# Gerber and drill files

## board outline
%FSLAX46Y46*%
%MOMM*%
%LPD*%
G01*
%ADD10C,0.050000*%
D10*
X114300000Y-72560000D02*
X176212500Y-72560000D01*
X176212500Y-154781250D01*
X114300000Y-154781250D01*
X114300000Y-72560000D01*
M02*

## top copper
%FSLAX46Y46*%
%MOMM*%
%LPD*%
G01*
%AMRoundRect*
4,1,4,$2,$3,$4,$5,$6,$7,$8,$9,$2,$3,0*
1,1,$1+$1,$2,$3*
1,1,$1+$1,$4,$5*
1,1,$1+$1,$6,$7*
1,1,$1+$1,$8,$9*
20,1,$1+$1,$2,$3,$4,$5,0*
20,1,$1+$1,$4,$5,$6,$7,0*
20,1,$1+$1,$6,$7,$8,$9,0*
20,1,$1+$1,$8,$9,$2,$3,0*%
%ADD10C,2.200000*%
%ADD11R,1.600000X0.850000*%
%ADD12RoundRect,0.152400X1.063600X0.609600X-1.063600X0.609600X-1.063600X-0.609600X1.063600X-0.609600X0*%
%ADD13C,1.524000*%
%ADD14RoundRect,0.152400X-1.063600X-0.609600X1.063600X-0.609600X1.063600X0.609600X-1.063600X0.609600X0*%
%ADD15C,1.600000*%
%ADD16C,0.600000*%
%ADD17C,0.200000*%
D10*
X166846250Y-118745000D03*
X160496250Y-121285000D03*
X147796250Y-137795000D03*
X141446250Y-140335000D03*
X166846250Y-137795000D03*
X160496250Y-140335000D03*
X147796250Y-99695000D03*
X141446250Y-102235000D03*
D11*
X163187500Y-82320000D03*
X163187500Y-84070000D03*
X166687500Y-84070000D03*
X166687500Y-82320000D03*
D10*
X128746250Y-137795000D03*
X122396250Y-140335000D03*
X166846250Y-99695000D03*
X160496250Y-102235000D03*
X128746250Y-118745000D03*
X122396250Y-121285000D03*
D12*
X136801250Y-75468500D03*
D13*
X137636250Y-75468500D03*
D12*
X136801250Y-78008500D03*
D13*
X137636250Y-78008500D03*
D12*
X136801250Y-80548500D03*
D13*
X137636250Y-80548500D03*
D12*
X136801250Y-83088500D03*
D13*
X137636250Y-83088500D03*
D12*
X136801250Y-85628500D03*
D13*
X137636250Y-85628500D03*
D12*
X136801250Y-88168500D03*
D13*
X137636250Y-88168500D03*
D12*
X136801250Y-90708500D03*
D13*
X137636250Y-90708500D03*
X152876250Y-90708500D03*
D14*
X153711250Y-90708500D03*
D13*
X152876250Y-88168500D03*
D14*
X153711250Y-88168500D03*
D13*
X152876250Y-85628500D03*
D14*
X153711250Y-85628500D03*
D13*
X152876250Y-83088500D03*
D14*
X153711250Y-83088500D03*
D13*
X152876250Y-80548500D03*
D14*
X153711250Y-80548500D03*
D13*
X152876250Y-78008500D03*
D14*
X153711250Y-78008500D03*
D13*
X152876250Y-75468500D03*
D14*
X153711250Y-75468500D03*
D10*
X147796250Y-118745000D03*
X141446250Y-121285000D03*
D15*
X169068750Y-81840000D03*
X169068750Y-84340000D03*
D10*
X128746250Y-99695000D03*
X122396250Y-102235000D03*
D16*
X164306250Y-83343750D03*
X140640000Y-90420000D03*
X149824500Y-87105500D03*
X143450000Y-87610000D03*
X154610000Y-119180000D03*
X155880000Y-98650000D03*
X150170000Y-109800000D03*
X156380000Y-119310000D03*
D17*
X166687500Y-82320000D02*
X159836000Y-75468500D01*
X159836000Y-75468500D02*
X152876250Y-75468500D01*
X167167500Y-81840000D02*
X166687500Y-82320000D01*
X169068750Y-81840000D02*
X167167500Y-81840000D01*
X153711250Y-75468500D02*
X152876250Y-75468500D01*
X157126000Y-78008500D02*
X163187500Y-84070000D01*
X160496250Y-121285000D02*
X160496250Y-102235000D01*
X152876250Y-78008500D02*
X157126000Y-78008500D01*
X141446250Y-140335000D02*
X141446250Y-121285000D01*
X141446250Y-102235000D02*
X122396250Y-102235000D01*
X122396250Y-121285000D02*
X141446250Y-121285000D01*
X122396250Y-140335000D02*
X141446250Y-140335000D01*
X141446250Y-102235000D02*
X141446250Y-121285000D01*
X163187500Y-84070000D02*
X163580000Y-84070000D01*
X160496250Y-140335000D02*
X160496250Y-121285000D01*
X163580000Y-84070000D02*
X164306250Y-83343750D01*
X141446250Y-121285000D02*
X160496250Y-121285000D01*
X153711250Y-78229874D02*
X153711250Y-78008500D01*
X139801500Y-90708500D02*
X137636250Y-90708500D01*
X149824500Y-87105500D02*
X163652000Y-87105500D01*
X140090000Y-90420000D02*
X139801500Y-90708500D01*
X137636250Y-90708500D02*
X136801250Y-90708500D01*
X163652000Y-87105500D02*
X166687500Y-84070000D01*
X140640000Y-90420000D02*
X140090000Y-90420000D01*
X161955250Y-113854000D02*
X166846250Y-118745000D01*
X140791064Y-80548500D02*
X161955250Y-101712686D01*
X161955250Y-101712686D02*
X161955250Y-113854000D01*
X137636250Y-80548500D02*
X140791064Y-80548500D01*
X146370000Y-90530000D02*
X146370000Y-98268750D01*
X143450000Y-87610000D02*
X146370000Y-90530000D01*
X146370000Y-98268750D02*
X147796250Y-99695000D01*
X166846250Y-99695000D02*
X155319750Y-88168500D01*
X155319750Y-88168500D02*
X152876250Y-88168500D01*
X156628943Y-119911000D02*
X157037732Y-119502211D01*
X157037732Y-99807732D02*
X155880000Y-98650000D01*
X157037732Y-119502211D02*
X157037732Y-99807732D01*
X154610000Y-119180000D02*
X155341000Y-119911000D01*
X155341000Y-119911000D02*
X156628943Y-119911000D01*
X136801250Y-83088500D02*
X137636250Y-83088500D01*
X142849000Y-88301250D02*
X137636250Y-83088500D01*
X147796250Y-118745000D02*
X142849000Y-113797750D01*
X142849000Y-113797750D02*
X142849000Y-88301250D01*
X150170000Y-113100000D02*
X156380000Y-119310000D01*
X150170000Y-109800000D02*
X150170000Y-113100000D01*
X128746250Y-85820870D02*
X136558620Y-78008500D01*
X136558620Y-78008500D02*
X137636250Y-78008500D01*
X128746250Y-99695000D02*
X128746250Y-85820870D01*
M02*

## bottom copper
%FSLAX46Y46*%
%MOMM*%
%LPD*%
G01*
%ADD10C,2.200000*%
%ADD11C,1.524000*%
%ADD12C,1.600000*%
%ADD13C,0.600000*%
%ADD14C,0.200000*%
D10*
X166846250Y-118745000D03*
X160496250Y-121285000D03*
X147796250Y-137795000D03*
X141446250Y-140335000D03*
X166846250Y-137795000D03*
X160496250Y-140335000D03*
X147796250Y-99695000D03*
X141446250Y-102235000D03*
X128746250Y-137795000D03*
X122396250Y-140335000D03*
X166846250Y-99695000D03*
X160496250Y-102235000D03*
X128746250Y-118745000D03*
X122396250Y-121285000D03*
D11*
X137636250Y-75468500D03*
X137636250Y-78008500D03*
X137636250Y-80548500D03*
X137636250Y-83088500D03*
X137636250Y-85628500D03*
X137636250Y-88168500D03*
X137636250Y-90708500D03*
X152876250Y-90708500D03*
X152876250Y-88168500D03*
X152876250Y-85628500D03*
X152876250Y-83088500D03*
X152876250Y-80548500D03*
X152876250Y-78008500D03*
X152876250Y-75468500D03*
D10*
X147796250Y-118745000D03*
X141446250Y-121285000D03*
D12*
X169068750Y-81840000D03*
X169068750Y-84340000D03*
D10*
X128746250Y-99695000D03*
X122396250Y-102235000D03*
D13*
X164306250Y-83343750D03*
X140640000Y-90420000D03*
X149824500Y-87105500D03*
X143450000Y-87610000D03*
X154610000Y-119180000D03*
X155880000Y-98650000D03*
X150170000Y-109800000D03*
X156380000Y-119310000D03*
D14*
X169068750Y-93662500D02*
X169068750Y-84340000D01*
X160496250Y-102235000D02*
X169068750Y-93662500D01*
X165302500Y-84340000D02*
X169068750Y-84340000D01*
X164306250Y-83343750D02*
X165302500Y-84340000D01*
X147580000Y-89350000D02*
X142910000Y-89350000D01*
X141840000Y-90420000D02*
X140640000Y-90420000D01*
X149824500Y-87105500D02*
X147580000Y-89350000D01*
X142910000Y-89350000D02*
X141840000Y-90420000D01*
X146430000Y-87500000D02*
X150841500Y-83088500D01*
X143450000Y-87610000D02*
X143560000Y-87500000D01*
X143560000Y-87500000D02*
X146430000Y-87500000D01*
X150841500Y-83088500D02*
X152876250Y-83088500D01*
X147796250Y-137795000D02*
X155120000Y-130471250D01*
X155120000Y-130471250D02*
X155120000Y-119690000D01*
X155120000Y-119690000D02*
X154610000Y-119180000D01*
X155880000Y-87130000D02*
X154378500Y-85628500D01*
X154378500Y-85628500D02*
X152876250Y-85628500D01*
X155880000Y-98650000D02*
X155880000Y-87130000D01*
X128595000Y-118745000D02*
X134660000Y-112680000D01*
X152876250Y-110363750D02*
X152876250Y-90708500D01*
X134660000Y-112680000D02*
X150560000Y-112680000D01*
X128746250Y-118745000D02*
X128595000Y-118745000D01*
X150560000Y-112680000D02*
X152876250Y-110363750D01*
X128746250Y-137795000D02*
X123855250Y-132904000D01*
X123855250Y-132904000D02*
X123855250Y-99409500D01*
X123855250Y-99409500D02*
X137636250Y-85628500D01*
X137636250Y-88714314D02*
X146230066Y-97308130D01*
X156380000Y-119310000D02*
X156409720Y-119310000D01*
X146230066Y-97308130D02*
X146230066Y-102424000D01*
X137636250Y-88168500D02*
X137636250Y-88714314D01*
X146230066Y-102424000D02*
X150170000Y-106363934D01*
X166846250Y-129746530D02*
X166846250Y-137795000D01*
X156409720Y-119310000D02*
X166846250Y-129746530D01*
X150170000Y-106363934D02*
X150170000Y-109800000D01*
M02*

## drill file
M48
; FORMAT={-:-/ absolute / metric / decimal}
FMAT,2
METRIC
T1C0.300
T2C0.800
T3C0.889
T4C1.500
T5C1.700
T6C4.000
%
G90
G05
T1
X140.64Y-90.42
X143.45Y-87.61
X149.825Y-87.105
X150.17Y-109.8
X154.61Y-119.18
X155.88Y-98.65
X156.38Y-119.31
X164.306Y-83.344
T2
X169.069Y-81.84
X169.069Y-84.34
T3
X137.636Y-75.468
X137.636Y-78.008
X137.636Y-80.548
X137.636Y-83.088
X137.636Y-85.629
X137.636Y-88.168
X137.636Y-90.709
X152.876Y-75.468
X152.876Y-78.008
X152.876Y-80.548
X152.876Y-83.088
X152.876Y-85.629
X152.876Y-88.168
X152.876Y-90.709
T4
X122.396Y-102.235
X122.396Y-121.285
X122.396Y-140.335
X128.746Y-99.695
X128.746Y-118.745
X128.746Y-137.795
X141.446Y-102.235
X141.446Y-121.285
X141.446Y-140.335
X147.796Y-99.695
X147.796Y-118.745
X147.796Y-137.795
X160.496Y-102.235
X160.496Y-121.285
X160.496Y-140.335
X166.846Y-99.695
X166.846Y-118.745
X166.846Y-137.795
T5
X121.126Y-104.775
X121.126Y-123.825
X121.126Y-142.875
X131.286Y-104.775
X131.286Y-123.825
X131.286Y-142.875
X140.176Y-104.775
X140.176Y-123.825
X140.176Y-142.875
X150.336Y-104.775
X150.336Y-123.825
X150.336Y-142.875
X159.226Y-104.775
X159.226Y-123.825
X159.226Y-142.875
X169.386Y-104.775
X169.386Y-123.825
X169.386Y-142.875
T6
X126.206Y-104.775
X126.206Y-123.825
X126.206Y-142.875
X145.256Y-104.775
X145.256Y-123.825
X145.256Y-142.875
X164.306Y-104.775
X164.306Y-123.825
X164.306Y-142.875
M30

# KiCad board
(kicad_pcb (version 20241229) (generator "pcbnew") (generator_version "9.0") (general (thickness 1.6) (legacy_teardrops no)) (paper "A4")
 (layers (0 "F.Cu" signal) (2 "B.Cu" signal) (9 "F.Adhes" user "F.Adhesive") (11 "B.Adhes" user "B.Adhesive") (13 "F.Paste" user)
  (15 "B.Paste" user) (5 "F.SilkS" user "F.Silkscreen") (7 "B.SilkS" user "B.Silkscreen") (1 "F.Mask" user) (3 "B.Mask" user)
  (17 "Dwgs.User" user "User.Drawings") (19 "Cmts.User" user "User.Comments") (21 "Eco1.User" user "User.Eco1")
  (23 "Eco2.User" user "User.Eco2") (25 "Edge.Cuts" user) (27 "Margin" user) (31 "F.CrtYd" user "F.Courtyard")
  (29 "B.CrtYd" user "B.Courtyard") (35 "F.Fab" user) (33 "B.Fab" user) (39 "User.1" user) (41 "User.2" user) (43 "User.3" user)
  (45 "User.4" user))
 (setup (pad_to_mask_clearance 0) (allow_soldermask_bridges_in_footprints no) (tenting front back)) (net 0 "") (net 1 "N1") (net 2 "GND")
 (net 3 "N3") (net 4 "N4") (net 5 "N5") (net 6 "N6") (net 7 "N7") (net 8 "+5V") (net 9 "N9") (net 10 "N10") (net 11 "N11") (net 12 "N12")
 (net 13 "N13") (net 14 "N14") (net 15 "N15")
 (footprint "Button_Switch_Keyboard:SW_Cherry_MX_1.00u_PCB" (layer "F.Cu") (at 166.84625 118.745)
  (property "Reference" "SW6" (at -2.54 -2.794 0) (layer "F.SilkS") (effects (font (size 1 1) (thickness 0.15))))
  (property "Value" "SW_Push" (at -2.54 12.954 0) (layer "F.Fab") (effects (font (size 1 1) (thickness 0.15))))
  (pad "" np_thru_hole circle (at -7.62 5.08) (size 1.7 1.7) (drill 1.7) (layers "*.Cu" "*.Mask"))
  (pad "" np_thru_hole circle (at -2.54 5.08) (size 4 4) (drill 4) (layers "*.Cu" "*.Mask"))
  (pad "" np_thru_hole circle (at 2.54 5.08) (size 1.7 1.7) (drill 1.7) (layers "*.Cu" "*.Mask"))
  (pad "1" thru_hole circle (at 0 0) (size 2.2 2.2) (drill 1.5) (layers "*.Cu" "*.Mask") (remove_unused_layers no) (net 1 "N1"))
  (pad "2" thru_hole circle (at -6.35 2.54) (size 2.2 2.2) (drill 1.5) (layers "*.Cu" "*.Mask") (remove_unused_layers no) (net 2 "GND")))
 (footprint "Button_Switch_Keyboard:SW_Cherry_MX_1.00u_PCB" (layer "F.Cu") (at 147.79625 137.795)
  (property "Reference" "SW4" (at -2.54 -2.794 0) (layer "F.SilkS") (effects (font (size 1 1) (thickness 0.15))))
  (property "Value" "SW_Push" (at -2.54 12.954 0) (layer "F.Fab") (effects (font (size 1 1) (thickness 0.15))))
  (pad "" np_thru_hole circle (at -7.62 5.08) (size 1.7 1.7) (drill 1.7) (layers "*.Cu" "*.Mask"))
  (pad "" np_thru_hole circle (at -2.54 5.08) (size 4 4) (drill 4) (layers "*.Cu" "*.Mask"))
  (pad "" np_thru_hole circle (at 2.54 5.08) (size 1.7 1.7) (drill 1.7) (layers "*.Cu" "*.Mask"))
  (pad "1" thru_hole circle (at 0 0) (size 2.2 2.2) (drill 1.5) (layers "*.Cu" "*.Mask") (remove_unused_layers no) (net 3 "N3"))
  (pad "2" thru_hole circle (at -6.35 2.54) (size 2.2 2.2) (drill 1.5) (layers "*.Cu" "*.Mask") (remove_unused_layers no) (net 2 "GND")))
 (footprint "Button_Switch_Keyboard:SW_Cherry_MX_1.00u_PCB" (layer "F.Cu") (at 166.84625 137.795)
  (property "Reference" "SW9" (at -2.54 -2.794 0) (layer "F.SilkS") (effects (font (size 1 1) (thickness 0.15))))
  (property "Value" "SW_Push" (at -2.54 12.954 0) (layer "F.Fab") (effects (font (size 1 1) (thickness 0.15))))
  (pad "" np_thru_hole circle (at -7.62 5.08) (size 1.7 1.7) (drill 1.7) (layers "*.Cu" "*.Mask"))
  (pad "" np_thru_hole circle (at -2.54 5.08) (size 4 4) (drill 4) (layers "*.Cu" "*.Mask"))
  (pad "" np_thru_hole circle (at 2.54 5.08) (size 1.7 1.7) (drill 1.7) (layers "*.Cu" "*.Mask"))
  (pad "1" thru_hole circle (at 0 0) (size 2.2 2.2) (drill 1.5) (layers "*.Cu" "*.Mask") (remove_unused_layers no) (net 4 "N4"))
  (pad "2" thru_hole circle (at -6.35 2.54) (size 2.2 2.2) (drill 1.5) (layers "*.Cu" "*.Mask") (remove_unused_layers no) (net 2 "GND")))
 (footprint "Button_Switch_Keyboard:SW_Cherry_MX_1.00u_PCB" (layer "F.Cu") (at 147.79625 99.695)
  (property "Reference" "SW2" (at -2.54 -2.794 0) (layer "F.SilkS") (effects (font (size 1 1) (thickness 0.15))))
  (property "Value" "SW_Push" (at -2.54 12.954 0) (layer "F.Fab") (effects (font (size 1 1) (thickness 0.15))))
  (pad "" np_thru_hole circle (at -7.62 5.08) (size 1.7 1.7) (drill 1.7) (layers "*.Cu" "*.Mask"))
  (pad "" np_thru_hole circle (at -2.54 5.08) (size 4 4) (drill 4) (layers "*.Cu" "*.Mask"))
  (pad "" np_thru_hole circle (at 2.54 5.08) (size 1.7 1.7) (drill 1.7) (layers "*.Cu" "*.Mask"))
  (pad "1" thru_hole circle (at 0 0) (size 2.2 2.2) (drill 1.5) (layers "*.Cu" "*.Mask") (remove_unused_layers no) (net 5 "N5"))
  (pad "2" thru_hole circle (at -6.35 2.54) (size 2.2 2.2) (drill 1.5) (layers "*.Cu" "*.Mask") (remove_unused_layers no) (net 2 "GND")))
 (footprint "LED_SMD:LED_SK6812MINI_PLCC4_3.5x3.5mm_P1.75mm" (layer "F.Cu") (at 164.9375 83.195)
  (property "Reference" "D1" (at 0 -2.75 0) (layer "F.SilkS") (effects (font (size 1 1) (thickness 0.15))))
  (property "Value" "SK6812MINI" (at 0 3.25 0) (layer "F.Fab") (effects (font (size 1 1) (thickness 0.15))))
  (pad "1" smd rect (at -1.75 -0.875) (size 1.6 0.85) (layers "F.Cu" "F.Mask" "F.Paste") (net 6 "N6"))
  (pad "2" smd rect (at -1.75 0.875) (size 1.6 0.85) (layers "F.Cu" "F.Mask" "F.Paste") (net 2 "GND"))
  (pad "3" smd rect (at 1.75 0.875) (size 1.6 0.85) (layers "F.Cu" "F.Mask" "F.Paste") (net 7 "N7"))
  (pad "4" smd rect (at 1.75 -0.875) (size 1.6 0.85) (layers "F.Cu" "F.Mask" "F.Paste") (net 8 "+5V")))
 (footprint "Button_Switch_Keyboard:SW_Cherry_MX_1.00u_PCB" (layer "F.Cu") (at 128.74625 137.795)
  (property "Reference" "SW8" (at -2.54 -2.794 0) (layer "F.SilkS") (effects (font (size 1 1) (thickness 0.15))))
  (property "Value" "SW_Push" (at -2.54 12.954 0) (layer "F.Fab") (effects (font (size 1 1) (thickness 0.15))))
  (pad "" np_thru_hole circle (at -7.62 5.08) (size 1.7 1.7) (drill 1.7) (layers "*.Cu" "*.Mask"))
  (pad "" np_thru_hole circle (at -2.54 5.08) (size 4 4) (drill 4) (layers "*.Cu" "*.Mask"))
  (pad "" np_thru_hole circle (at 2.54 5.08) (size 1.7 1.7) (drill 1.7) (layers "*.Cu" "*.Mask"))
  (pad "1" thru_hole circle (at 0 0) (size 2.2 2.2) (drill 1.5) (layers "*.Cu" "*.Mask") (remove_unused_layers no) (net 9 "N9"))
  (pad "2" thru_hole circle (at -6.35 2.54) (size 2.2 2.2) (drill 1.5) (layers "*.Cu" "*.Mask") (remove_unused_layers no) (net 2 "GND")))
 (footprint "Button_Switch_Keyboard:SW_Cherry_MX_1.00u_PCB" (layer "F.Cu") (at 166.84625 99.695)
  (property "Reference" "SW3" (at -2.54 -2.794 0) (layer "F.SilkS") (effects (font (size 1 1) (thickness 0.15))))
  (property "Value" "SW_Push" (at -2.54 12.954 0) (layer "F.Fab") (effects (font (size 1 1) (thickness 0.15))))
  (pad "" np_thru_hole circle (at -7.62 5.08) (size 1.7 1.7) (drill 1.7) (layers "*.Cu" "*.Mask"))
  (pad "" np_thru_hole circle (at -2.54 5.08) (size 4 4) (drill 4) (layers "*.Cu" "*.Mask"))
  (pad "" np_thru_hole circle (at 2.54 5.08) (size 1.7 1.7) (drill 1.7) (layers "*.Cu" "*.Mask"))
  (pad "1" thru_hole circle (at 0 0) (size 2.2 2.2) (drill 1.5) (layers "*.Cu" "*.Mask") (remove_unused_layers no) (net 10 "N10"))
  (pad "2" thru_hole circle (at -6.35 2.54) (size 2.2 2.2) (drill 1.5) (layers "*.Cu" "*.Mask") (remove_unused_layers no) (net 2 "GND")))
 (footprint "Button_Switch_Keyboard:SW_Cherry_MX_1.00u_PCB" (layer "F.Cu") (at 128.74625 118.745)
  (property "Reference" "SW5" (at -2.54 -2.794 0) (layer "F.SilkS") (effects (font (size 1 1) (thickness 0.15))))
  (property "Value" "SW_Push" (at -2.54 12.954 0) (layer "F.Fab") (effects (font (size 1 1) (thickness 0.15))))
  (pad "" np_thru_hole circle (at -7.62 5.08) (size 1.7 1.7) (drill 1.7) (layers "*.Cu" "*.Mask"))
  (pad "" np_thru_hole circle (at -2.54 5.08) (size 4 4) (drill 4) (layers "*.Cu" "*.Mask"))
  (pad "" np_thru_hole circle (at 2.54 5.08) (size 1.7 1.7) (drill 1.7) (layers "*.Cu" "*.Mask"))
  (pad "1" thru_hole circle (at 0 0) (size 2.2 2.2) (drill 1.5) (layers "*.Cu" "*.Mask") (remove_unused_layers no) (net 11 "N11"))
  (pad "2" thru_hole circle (at -6.35 2.54) (size 2.2 2.2) (drill 1.5) (layers "*.Cu" "*.Mask") (remove_unused_layers no) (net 2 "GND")))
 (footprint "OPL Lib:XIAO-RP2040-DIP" (layer "F.Cu") (at 145.25625 83.0885)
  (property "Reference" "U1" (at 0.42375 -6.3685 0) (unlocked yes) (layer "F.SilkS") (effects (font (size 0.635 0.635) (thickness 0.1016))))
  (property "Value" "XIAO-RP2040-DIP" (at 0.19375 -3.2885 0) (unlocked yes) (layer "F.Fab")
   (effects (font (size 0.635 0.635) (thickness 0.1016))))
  (pad "1" smd roundrect (at -8.455 -7.62 180) (size 2.432 1.524) (layers "F.Cu" "F.Mask") (roundrect_rratio 0.1) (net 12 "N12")
   (thermal_bridge_angle 45))
  (pad "1" thru_hole circle (at -7.62 -7.62 180) (size 1.524 1.524) (drill 0.889) (layers "*.Cu" "*.Mask") (remove_unused_layers no)
   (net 12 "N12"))
  (pad "2" smd roundrect (at -8.455 -5.08 180) (size 2.432 1.524) (layers "F.Cu" "F.Mask") (roundrect_rratio 0.1) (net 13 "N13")
   (thermal_bridge_angle 45))
  (pad "2" thru_hole circle (at -7.62 -5.08 180) (size 1.524 1.524) (drill 0.889) (layers "*.Cu" "*.Mask") (remove_unused_layers no)
   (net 13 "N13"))
  (pad "3" smd roundrect (at -8.455 -2.54 180) (size 2.432 1.524) (layers "F.Cu" "F.Mask") (roundrect_rratio 0.1) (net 1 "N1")
   (thermal_bridge_angle 45))
  (pad "3" thru_hole circle (at -7.62 -2.54 180) (size 1.524 1.524) (drill 0.889) (layers "*.Cu" "*.Mask") (remove_unused_layers no)
   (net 1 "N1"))
  (pad "4" smd roundrect (at -8.455 0 180) (size 2.432 1.524) (layers "F.Cu" "F.Mask") (roundrect_rratio 0.1) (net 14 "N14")
   (thermal_bridge_angle 45))
  (pad "4" thru_hole circle (at -7.62 0 180) (size 1.524 1.524) (drill 0.889) (layers "*.Cu" "*.Mask") (remove_unused_layers no)
   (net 14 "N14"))
  (pad "5" smd roundrect (at -8.455 2.54 180) (size 2.432 1.524) (layers "F.Cu" "F.Mask") (roundrect_rratio 0.1) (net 9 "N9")
   (thermal_bridge_angle 45))
  (pad "5" thru_hole circle (at -7.62 2.54 180) (size 1.524 1.524) (drill 0.889) (layers "*.Cu" "*.Mask") (remove_unused_layers no)
   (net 9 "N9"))
  (pad "6" smd roundrect (at -8.455 5.08 180) (size 2.432 1.524) (layers "F.Cu" "F.Mask") (roundrect_rratio 0.1) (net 4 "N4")
   (thermal_bridge_angle 45))
  (pad "6" thru_hole circle (at -7.62 5.08 180) (size 1.524 1.524) (drill 0.889) (layers "*.Cu" "*.Mask") (remove_unused_layers no)
   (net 4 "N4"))
  (pad "7" smd roundrect (at -8.455 7.62 180) (size 2.432 1.524) (layers "F.Cu" "F.Mask") (roundrect_rratio 0.1) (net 7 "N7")
   (thermal_bridge_angle 45))
  (pad "7" thru_hole circle (at -7.62 7.62 180) (size 1.524 1.524) (drill 0.889) (layers "*.Cu" "*.Mask") (remove_unused_layers no)
   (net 7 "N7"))
  (pad "8" thru_hole circle (at 7.62 7.62) (size 1.524 1.524) (drill 0.889) (layers "*.Cu" "*.Mask") (remove_unused_layers no)
   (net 11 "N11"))
  (pad "8" smd roundrect (at 8.455 7.62) (size 2.432 1.524) (layers "F.Cu" "F.Mask") (roundrect_rratio 0.1) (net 11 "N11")
   (thermal_bridge_angle 45))
  (pad "9" thru_hole circle (at 7.62 5.08) (size 1.524 1.524) (drill 0.889) (layers "*.Cu" "*.Mask") (remove_unused_layers no)
   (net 10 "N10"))
  (pad "9" smd roundrect (at 8.455 5.08) (size 2.432 1.524) (layers "F.Cu" "F.Mask") (roundrect_rratio 0.1) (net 10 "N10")
   (thermal_bridge_angle 45))
  (pad "10" thru_hole circle (at 7.62 2.54) (size 1.524 1.524) (drill 0.889) (layers "*.Cu" "*.Mask") (remove_unused_layers no) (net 3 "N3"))
  (pad "10" smd roundrect (at 8.455 2.54) (size 2.432 1.524) (layers "F.Cu" "F.Mask") (roundrect_rratio 0.1) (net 3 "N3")
   (thermal_bridge_angle 45))
  (pad "11" thru_hole circle (at 7.62 0) (size 1.524 1.524) (drill 0.889) (layers "*.Cu" "*.Mask") (remove_unused_layers no) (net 5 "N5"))
  (pad "11" smd roundrect (at 8.455 0) (size 2.432 1.524) (layers "F.Cu" "F.Mask") (roundrect_rratio 0.1) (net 5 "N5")
   (thermal_bridge_angle 45))
  (pad "12" thru_hole circle (at 7.62 -2.54) (size 1.524 1.524) (drill 0.889) (layers "*.Cu" "*.Mask") (remove_unused_layers no)
   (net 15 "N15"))
  (pad "12" smd roundrect (at 8.455 -2.54) (size 2.432 1.524) (layers "F.Cu" "F.Mask") (roundrect_rratio 0.1) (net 15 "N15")
   (thermal_bridge_angle 45))
  (pad "13" thru_hole circle (at 7.62 -5.08) (size 1.524 1.524) (drill 0.889) (layers "*.Cu" "*.Mask") (remove_unused_layers no)
   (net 2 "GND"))
  (pad "13" smd roundrect (at 8.455 -5.08) (size 2.432 1.524) (layers "F.Cu" "F.Mask") (roundrect_rratio 0.1) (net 2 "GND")
   (thermal_bridge_angle 45))
  (pad "14" thru_hole circle (at 7.62 -7.62) (size 1.524 1.524) (drill 0.889) (layers "*.Cu" "*.Mask") (remove_unused_layers no)
   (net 8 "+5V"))
  (pad "14" smd roundrect (at 8.455 -7.62) (size 2.432 1.524) (layers "F.Cu" "F.Mask") (roundrect_rratio 0.1) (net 8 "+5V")
   (thermal_bridge_angle 45)))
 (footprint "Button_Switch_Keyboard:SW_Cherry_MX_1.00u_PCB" (layer "F.Cu") (at 147.79625 118.745)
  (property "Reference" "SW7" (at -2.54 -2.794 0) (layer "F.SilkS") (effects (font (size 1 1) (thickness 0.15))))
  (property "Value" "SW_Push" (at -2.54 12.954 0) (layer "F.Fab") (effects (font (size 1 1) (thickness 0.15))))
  (pad "" np_thru_hole circle (at -7.62 5.08) (size 1.7 1.7) (drill 1.7) (layers "*.Cu" "*.Mask"))
  (pad "" np_thru_hole circle (at -2.54 5.08) (size 4 4) (drill 4) (layers "*.Cu" "*.Mask"))
  (pad "" np_thru_hole circle (at 2.54 5.08) (size 1.7 1.7) (drill 1.7) (layers "*.Cu" "*.Mask"))
  (pad "1" thru_hole circle (at 0 0) (size 2.2 2.2) (drill 1.5) (layers "*.Cu" "*.Mask") (remove_unused_layers no) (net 14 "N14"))
  (pad "2" thru_hole circle (at -6.35 2.54) (size 2.2 2.2) (drill 1.5) (layers "*.Cu" "*.Mask") (remove_unused_layers no) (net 2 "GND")))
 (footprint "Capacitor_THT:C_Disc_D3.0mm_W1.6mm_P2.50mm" (layer "F.Cu") (at 169.06875 81.84 -90)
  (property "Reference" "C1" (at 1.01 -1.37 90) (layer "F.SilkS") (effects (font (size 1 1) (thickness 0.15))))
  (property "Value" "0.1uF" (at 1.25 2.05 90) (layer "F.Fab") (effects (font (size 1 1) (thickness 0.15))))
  (pad "1" thru_hole circle (at 0 0 270) (size 1.6 1.6) (drill 0.8) (layers "*.Cu" "*.Mask") (remove_unused_layers no) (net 8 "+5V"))
  (pad "2" thru_hole circle (at 2.5 0 270) (size 1.6 1.6) (drill 0.8) (layers "*.Cu" "*.Mask") (remove_unused_layers no) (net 2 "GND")))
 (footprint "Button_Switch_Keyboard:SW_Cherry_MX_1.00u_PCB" (layer "F.Cu") (at 128.74625 99.695)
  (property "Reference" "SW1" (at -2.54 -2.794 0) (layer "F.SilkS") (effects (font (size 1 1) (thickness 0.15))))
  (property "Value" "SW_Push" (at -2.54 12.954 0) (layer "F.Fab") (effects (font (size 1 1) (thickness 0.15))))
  (pad "" np_thru_hole circle (at -7.62 5.08) (size 1.7 1.7) (drill 1.7) (layers "*.Cu" "*.Mask"))
  (pad "" np_thru_hole circle (at -2.54 5.08) (size 4 4) (drill 4) (layers "*.Cu" "*.Mask"))
  (pad "" np_thru_hole circle (at 2.54 5.08) (size 1.7 1.7) (drill 1.7) (layers "*.Cu" "*.Mask"))
  (pad "1" thru_hole circle (at 0 0) (size 2.2 2.2) (drill 1.5) (layers "*.Cu" "*.Mask") (remove_unused_layers no) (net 13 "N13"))
  (pad "2" thru_hole circle (at -6.35 2.54) (size 2.2 2.2) (drill 1.5) (layers "*.Cu" "*.Mask") (remove_unused_layers no) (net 2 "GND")))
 (gr_rect (start 114.3 72.56) (end 176.2125 154.78125) (stroke (width 0.05) (type default)) (fill no) (layer "Edge.Cuts"))
 (segment (start 166.6875 82.32) (end 159.836 75.4685) (width 0.2) (layer "F.Cu") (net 8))
 (segment (start 159.836 75.4685) (end 152.87625 75.4685) (width 0.2) (layer "F.Cu") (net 8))
 (segment (start 167.1675 81.84) (end 166.6875 82.32) (width 0.2) (layer "F.Cu") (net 8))
 (segment (start 169.06875 81.84) (end 167.1675 81.84) (width 0.2) (layer "F.Cu") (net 8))
 (segment (start 153.71125 75.4685) (end 152.87625 75.4685) (width 0.2) (layer "F.Cu") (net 8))
 (segment (start 157.126 78.0085) (end 163.1875 84.07) (width 0.2) (layer "F.Cu") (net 2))
 (segment (start 160.49625 121.285) (end 160.49625 102.235) (width 0.2) (layer "F.Cu") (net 2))
 (segment (start 152.87625 78.0085) (end 157.126 78.0085) (width 0.2) (layer "F.Cu") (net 2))
 (segment (start 141.44625 140.335) (end 141.44625 121.285) (width 0.2) (layer "F.Cu") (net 2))
 (segment (start 141.44625 102.235) (end 122.39625 102.235) (width 0.2) (layer "F.Cu") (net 2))
 (segment (start 122.39625 121.285) (end 141.44625 121.285) (width 0.2) (layer "F.Cu") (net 2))
 (segment (start 122.39625 140.335) (end 141.44625 140.335) (width 0.2) (layer "F.Cu") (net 2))
 (segment (start 141.44625 102.235) (end 141.44625 121.285) (width 0.2) (layer "F.Cu") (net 2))
 (segment (start 163.1875 84.07) (end 163.58 84.07) (width 0.2) (layer "F.Cu") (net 2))
 (segment (start 160.49625 140.335) (end 160.49625 121.285) (width 0.2) (layer "F.Cu") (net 2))
 (segment (start 163.58 84.07) (end 164.30625 83.34375) (width 0.2) (layer "F.Cu") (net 2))
 (segment (start 141.44625 121.285) (end 160.49625 121.285) (width 0.2) (layer "F.Cu") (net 2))
 (segment (start 153.71125 78.229874) (end 153.71125 78.0085) (width 0.2) (layer "F.Cu") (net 2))
 (via (at 164.30625 83.34375) (size 0.6) (drill 0.3) (layers "F.Cu" "B.Cu") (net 2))
 (segment (start 169.06875 93.6625) (end 169.06875 84.34) (width 0.2) (layer "B.Cu") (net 2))
 (segment (start 160.49625 102.235) (end 169.06875 93.6625) (width 0.2) (layer "B.Cu") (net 2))
 (segment (start 165.3025 84.34) (end 169.06875 84.34) (width 0.2) (layer "B.Cu") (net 2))
 (segment (start 164.30625 83.34375) (end 165.3025 84.34) (width 0.2) (layer "B.Cu") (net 2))
 (segment (start 139.8015 90.7085) (end 137.63625 90.7085) (width 0.2) (layer "F.Cu") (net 7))
 (segment (start 149.8245 87.1055) (end 163.652 87.1055) (width 0.2) (layer "F.Cu") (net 7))
 (segment (start 140.09 90.42) (end 139.8015 90.7085) (width 0.2) (layer "F.Cu") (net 7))
 (segment (start 137.63625 90.7085) (end 136.80125 90.7085) (width 0.2) (layer "F.Cu") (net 7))
 (segment (start 163.652 87.1055) (end 166.6875 84.07) (width 0.2) (layer "F.Cu") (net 7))
 (segment (start 140.64 90.42) (end 140.09 90.42) (width 0.2) (layer "F.Cu") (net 7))
 (via (at 140.64 90.42) (size 0.6) (drill 0.3) (layers "F.Cu" "B.Cu") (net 7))
 (via (at 149.8245 87.1055) (size 0.6) (drill 0.3) (layers "F.Cu" "B.Cu") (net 7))
 (segment (start 147.58 89.35) (end 142.91 89.35) (width 0.2) (layer "B.Cu") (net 7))
 (segment (start 141.84 90.42) (end 140.64 90.42) (width 0.2) (layer "B.Cu") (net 7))
 (segment (start 149.8245 87.1055) (end 147.58 89.35) (width 0.2) (layer "B.Cu") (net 7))
 (segment (start 142.91 89.35) (end 141.84 90.42) (width 0.2) (layer "B.Cu") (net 7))
 (segment (start 161.95525 113.854) (end 166.84625 118.745) (width 0.2) (layer "F.Cu") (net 1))
 (segment (start 140.791064 80.5485) (end 161.95525 101.712686) (width 0.2) (layer "F.Cu") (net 1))
 (segment (start 161.95525 101.712686) (end 161.95525 113.854) (width 0.2) (layer "F.Cu") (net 1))
 (segment (start 137.63625 80.5485) (end 140.791064 80.5485) (width 0.2) (layer "F.Cu") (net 1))
 (segment (start 146.37 90.53) (end 146.37 98.26875) (width 0.2) (layer "F.Cu") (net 5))
 (segment (start 143.45 87.61) (end 146.37 90.53) (width 0.2) (layer "F.Cu") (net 5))
 (segment (start 146.37 98.26875) (end 147.79625 99.695) (width 0.2) (layer "F.Cu") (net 5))
 (via (at 143.45 87.61) (size 0.6) (drill 0.3) (layers "F.Cu" "B.Cu") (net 5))
 (segment (start 146.43 87.5) (end 150.8415 83.0885) (width 0.2) (layer "B.Cu") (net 5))
 (segment (start 143.45 87.61) (end 143.56 87.5) (width 0.2) (layer "B.Cu") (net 5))
 (segment (start 143.56 87.5) (end 146.43 87.5) (width 0.2) (layer "B.Cu") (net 5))
 (segment (start 150.8415 83.0885) (end 152.87625 83.0885) (width 0.2) (layer "B.Cu") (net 5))
 (segment (start 166.84625 99.695) (end 155.31975 88.1685) (width 0.2) (layer "F.Cu") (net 10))
 (segment (start 155.31975 88.1685) (end 152.87625 88.1685) (width 0.2) (layer "F.Cu") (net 10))
 (segment (start 156.628943 119.911) (end 157.037732 119.502211) (width 0.2) (layer "F.Cu") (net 3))
 (segment (start 157.037732 99.807732) (end 155.88 98.65) (width 0.2) (layer "F.Cu") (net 3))
 (segment (start 157.037732 119.502211) (end 157.037732 99.807732) (width 0.2) (layer "F.Cu") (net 3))
 (segment (start 154.61 119.18) (end 155.341 119.911) (width 0.2) (layer "F.Cu") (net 3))
 (segment (start 155.341 119.911) (end 156.628943 119.911) (width 0.2) (layer "F.Cu") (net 3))
 (via (at 154.61 119.18) (size 0.6) (drill 0.3) (layers "F.Cu" "B.Cu") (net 3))
 (via (at 155.88 98.65) (size 0.6) (drill 0.3) (layers "F.Cu" "B.Cu") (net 3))
 (segment (start 147.79625 137.795) (end 155.12 130.47125) (width 0.2) (layer "B.Cu") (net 3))
 (segment (start 155.12 130.47125) (end 155.12 119.69) (width 0.2) (layer "B.Cu") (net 3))
 (segment (start 155.12 119.69) (end 154.61 119.18) (width 0.2) (layer "B.Cu") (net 3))
 (segment (start 155.88 87.13) (end 154.3785 85.6285) (width 0.2) (layer "B.Cu") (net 3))
 (segment (start 154.3785 85.6285) (end 152.87625 85.6285) (width 0.2) (layer "B.Cu") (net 3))
 (segment (start 155.88 98.65) (end 155.88 87.13) (width 0.2) (layer "B.Cu") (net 3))
 (segment (start 128.595 118.745) (end 134.66 112.68) (width 0.2) (layer "B.Cu") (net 11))
 (segment (start 152.87625 110.36375) (end 152.87625 90.7085) (width 0.2) (layer "B.Cu") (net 11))
 (segment (start 134.66 112.68) (end 150.56 112.68) (width 0.2) (layer "B.Cu") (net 11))
 (segment (start 128.74625 118.745) (end 128.595 118.745) (width 0.2) (layer "B.Cu") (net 11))
 (segment (start 150.56 112.68) (end 152.87625 110.36375) (width 0.2) (layer "B.Cu") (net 11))
 (segment (start 136.80125 83.0885) (end 137.63625 83.0885) (width 0.2) (layer "F.Cu") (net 14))
 (segment (start 142.849 88.30125) (end 137.63625 83.0885) (width 0.2) (layer "F.Cu") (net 14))
 (segment (start 147.79625 118.745) (end 142.849 113.79775) (width 0.2) (layer "F.Cu") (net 14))
 (segment (start 142.849 113.79775) (end 142.849 88.30125) (width 0.2) (layer "F.Cu") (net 14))
 (segment (start 128.74625 137.795) (end 123.85525 132.904) (width 0.2) (layer "B.Cu") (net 9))
 (segment (start 123.85525 132.904) (end 123.85525 99.4095) (width 0.2) (layer "B.Cu") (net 9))
 (segment (start 123.85525 99.4095) (end 137.63625 85.6285) (width 0.2) (layer "B.Cu") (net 9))
 (segment (start 150.17 113.1) (end 156.38 119.31) (width 0.2) (layer "F.Cu") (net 4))
 (segment (start 150.17 109.8) (end 150.17 113.1) (width 0.2) (layer "F.Cu") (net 4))
 (via (at 150.17 109.8) (size 0.6) (drill 0.3) (layers "F.Cu" "B.Cu") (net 4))
 (via (at 156.38 119.31) (size 0.6) (drill 0.3) (layers "F.Cu" "B.Cu") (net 4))
 (segment (start 137.63625 88.714314) (end 146.230066 97.30813) (width 0.2) (layer "B.Cu") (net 4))
 (segment (start 156.38 119.31) (end 156.40972 119.31) (width 0.2) (layer "B.Cu") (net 4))
 (segment (start 146.230066 97.30813) (end 146.230066 102.424) (width 0.2) (layer "B.Cu") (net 4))
 (segment (start 137.63625 88.1685) (end 137.63625 88.714314) (width 0.2) (layer "B.Cu") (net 4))
 (segment (start 146.230066 102.424) (end 150.17 106.363934) (width 0.2) (layer "B.Cu") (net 4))
 (segment (start 166.84625 129.74653) (end 166.84625 137.795) (width 0.2) (layer "B.Cu") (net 4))
 (segment (start 156.40972 119.31) (end 166.84625 129.74653) (width 0.2) (layer "B.Cu") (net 4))
 (segment (start 150.17 106.363934) (end 150.17 109.8) (width 0.2) (layer "B.Cu") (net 4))
 (segment (start 128.74625 85.82087) (end 136.55862 78.0085) (width 0.2) (layer "F.Cu") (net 13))
 (segment (start 136.55862 78.0085) (end 137.63625 78.0085) (width 0.2) (layer "F.Cu") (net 13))
 (segment (start 128.74625 99.695) (end 128.74625 85.82087) (width 0.2) (layer "F.Cu") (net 13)))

